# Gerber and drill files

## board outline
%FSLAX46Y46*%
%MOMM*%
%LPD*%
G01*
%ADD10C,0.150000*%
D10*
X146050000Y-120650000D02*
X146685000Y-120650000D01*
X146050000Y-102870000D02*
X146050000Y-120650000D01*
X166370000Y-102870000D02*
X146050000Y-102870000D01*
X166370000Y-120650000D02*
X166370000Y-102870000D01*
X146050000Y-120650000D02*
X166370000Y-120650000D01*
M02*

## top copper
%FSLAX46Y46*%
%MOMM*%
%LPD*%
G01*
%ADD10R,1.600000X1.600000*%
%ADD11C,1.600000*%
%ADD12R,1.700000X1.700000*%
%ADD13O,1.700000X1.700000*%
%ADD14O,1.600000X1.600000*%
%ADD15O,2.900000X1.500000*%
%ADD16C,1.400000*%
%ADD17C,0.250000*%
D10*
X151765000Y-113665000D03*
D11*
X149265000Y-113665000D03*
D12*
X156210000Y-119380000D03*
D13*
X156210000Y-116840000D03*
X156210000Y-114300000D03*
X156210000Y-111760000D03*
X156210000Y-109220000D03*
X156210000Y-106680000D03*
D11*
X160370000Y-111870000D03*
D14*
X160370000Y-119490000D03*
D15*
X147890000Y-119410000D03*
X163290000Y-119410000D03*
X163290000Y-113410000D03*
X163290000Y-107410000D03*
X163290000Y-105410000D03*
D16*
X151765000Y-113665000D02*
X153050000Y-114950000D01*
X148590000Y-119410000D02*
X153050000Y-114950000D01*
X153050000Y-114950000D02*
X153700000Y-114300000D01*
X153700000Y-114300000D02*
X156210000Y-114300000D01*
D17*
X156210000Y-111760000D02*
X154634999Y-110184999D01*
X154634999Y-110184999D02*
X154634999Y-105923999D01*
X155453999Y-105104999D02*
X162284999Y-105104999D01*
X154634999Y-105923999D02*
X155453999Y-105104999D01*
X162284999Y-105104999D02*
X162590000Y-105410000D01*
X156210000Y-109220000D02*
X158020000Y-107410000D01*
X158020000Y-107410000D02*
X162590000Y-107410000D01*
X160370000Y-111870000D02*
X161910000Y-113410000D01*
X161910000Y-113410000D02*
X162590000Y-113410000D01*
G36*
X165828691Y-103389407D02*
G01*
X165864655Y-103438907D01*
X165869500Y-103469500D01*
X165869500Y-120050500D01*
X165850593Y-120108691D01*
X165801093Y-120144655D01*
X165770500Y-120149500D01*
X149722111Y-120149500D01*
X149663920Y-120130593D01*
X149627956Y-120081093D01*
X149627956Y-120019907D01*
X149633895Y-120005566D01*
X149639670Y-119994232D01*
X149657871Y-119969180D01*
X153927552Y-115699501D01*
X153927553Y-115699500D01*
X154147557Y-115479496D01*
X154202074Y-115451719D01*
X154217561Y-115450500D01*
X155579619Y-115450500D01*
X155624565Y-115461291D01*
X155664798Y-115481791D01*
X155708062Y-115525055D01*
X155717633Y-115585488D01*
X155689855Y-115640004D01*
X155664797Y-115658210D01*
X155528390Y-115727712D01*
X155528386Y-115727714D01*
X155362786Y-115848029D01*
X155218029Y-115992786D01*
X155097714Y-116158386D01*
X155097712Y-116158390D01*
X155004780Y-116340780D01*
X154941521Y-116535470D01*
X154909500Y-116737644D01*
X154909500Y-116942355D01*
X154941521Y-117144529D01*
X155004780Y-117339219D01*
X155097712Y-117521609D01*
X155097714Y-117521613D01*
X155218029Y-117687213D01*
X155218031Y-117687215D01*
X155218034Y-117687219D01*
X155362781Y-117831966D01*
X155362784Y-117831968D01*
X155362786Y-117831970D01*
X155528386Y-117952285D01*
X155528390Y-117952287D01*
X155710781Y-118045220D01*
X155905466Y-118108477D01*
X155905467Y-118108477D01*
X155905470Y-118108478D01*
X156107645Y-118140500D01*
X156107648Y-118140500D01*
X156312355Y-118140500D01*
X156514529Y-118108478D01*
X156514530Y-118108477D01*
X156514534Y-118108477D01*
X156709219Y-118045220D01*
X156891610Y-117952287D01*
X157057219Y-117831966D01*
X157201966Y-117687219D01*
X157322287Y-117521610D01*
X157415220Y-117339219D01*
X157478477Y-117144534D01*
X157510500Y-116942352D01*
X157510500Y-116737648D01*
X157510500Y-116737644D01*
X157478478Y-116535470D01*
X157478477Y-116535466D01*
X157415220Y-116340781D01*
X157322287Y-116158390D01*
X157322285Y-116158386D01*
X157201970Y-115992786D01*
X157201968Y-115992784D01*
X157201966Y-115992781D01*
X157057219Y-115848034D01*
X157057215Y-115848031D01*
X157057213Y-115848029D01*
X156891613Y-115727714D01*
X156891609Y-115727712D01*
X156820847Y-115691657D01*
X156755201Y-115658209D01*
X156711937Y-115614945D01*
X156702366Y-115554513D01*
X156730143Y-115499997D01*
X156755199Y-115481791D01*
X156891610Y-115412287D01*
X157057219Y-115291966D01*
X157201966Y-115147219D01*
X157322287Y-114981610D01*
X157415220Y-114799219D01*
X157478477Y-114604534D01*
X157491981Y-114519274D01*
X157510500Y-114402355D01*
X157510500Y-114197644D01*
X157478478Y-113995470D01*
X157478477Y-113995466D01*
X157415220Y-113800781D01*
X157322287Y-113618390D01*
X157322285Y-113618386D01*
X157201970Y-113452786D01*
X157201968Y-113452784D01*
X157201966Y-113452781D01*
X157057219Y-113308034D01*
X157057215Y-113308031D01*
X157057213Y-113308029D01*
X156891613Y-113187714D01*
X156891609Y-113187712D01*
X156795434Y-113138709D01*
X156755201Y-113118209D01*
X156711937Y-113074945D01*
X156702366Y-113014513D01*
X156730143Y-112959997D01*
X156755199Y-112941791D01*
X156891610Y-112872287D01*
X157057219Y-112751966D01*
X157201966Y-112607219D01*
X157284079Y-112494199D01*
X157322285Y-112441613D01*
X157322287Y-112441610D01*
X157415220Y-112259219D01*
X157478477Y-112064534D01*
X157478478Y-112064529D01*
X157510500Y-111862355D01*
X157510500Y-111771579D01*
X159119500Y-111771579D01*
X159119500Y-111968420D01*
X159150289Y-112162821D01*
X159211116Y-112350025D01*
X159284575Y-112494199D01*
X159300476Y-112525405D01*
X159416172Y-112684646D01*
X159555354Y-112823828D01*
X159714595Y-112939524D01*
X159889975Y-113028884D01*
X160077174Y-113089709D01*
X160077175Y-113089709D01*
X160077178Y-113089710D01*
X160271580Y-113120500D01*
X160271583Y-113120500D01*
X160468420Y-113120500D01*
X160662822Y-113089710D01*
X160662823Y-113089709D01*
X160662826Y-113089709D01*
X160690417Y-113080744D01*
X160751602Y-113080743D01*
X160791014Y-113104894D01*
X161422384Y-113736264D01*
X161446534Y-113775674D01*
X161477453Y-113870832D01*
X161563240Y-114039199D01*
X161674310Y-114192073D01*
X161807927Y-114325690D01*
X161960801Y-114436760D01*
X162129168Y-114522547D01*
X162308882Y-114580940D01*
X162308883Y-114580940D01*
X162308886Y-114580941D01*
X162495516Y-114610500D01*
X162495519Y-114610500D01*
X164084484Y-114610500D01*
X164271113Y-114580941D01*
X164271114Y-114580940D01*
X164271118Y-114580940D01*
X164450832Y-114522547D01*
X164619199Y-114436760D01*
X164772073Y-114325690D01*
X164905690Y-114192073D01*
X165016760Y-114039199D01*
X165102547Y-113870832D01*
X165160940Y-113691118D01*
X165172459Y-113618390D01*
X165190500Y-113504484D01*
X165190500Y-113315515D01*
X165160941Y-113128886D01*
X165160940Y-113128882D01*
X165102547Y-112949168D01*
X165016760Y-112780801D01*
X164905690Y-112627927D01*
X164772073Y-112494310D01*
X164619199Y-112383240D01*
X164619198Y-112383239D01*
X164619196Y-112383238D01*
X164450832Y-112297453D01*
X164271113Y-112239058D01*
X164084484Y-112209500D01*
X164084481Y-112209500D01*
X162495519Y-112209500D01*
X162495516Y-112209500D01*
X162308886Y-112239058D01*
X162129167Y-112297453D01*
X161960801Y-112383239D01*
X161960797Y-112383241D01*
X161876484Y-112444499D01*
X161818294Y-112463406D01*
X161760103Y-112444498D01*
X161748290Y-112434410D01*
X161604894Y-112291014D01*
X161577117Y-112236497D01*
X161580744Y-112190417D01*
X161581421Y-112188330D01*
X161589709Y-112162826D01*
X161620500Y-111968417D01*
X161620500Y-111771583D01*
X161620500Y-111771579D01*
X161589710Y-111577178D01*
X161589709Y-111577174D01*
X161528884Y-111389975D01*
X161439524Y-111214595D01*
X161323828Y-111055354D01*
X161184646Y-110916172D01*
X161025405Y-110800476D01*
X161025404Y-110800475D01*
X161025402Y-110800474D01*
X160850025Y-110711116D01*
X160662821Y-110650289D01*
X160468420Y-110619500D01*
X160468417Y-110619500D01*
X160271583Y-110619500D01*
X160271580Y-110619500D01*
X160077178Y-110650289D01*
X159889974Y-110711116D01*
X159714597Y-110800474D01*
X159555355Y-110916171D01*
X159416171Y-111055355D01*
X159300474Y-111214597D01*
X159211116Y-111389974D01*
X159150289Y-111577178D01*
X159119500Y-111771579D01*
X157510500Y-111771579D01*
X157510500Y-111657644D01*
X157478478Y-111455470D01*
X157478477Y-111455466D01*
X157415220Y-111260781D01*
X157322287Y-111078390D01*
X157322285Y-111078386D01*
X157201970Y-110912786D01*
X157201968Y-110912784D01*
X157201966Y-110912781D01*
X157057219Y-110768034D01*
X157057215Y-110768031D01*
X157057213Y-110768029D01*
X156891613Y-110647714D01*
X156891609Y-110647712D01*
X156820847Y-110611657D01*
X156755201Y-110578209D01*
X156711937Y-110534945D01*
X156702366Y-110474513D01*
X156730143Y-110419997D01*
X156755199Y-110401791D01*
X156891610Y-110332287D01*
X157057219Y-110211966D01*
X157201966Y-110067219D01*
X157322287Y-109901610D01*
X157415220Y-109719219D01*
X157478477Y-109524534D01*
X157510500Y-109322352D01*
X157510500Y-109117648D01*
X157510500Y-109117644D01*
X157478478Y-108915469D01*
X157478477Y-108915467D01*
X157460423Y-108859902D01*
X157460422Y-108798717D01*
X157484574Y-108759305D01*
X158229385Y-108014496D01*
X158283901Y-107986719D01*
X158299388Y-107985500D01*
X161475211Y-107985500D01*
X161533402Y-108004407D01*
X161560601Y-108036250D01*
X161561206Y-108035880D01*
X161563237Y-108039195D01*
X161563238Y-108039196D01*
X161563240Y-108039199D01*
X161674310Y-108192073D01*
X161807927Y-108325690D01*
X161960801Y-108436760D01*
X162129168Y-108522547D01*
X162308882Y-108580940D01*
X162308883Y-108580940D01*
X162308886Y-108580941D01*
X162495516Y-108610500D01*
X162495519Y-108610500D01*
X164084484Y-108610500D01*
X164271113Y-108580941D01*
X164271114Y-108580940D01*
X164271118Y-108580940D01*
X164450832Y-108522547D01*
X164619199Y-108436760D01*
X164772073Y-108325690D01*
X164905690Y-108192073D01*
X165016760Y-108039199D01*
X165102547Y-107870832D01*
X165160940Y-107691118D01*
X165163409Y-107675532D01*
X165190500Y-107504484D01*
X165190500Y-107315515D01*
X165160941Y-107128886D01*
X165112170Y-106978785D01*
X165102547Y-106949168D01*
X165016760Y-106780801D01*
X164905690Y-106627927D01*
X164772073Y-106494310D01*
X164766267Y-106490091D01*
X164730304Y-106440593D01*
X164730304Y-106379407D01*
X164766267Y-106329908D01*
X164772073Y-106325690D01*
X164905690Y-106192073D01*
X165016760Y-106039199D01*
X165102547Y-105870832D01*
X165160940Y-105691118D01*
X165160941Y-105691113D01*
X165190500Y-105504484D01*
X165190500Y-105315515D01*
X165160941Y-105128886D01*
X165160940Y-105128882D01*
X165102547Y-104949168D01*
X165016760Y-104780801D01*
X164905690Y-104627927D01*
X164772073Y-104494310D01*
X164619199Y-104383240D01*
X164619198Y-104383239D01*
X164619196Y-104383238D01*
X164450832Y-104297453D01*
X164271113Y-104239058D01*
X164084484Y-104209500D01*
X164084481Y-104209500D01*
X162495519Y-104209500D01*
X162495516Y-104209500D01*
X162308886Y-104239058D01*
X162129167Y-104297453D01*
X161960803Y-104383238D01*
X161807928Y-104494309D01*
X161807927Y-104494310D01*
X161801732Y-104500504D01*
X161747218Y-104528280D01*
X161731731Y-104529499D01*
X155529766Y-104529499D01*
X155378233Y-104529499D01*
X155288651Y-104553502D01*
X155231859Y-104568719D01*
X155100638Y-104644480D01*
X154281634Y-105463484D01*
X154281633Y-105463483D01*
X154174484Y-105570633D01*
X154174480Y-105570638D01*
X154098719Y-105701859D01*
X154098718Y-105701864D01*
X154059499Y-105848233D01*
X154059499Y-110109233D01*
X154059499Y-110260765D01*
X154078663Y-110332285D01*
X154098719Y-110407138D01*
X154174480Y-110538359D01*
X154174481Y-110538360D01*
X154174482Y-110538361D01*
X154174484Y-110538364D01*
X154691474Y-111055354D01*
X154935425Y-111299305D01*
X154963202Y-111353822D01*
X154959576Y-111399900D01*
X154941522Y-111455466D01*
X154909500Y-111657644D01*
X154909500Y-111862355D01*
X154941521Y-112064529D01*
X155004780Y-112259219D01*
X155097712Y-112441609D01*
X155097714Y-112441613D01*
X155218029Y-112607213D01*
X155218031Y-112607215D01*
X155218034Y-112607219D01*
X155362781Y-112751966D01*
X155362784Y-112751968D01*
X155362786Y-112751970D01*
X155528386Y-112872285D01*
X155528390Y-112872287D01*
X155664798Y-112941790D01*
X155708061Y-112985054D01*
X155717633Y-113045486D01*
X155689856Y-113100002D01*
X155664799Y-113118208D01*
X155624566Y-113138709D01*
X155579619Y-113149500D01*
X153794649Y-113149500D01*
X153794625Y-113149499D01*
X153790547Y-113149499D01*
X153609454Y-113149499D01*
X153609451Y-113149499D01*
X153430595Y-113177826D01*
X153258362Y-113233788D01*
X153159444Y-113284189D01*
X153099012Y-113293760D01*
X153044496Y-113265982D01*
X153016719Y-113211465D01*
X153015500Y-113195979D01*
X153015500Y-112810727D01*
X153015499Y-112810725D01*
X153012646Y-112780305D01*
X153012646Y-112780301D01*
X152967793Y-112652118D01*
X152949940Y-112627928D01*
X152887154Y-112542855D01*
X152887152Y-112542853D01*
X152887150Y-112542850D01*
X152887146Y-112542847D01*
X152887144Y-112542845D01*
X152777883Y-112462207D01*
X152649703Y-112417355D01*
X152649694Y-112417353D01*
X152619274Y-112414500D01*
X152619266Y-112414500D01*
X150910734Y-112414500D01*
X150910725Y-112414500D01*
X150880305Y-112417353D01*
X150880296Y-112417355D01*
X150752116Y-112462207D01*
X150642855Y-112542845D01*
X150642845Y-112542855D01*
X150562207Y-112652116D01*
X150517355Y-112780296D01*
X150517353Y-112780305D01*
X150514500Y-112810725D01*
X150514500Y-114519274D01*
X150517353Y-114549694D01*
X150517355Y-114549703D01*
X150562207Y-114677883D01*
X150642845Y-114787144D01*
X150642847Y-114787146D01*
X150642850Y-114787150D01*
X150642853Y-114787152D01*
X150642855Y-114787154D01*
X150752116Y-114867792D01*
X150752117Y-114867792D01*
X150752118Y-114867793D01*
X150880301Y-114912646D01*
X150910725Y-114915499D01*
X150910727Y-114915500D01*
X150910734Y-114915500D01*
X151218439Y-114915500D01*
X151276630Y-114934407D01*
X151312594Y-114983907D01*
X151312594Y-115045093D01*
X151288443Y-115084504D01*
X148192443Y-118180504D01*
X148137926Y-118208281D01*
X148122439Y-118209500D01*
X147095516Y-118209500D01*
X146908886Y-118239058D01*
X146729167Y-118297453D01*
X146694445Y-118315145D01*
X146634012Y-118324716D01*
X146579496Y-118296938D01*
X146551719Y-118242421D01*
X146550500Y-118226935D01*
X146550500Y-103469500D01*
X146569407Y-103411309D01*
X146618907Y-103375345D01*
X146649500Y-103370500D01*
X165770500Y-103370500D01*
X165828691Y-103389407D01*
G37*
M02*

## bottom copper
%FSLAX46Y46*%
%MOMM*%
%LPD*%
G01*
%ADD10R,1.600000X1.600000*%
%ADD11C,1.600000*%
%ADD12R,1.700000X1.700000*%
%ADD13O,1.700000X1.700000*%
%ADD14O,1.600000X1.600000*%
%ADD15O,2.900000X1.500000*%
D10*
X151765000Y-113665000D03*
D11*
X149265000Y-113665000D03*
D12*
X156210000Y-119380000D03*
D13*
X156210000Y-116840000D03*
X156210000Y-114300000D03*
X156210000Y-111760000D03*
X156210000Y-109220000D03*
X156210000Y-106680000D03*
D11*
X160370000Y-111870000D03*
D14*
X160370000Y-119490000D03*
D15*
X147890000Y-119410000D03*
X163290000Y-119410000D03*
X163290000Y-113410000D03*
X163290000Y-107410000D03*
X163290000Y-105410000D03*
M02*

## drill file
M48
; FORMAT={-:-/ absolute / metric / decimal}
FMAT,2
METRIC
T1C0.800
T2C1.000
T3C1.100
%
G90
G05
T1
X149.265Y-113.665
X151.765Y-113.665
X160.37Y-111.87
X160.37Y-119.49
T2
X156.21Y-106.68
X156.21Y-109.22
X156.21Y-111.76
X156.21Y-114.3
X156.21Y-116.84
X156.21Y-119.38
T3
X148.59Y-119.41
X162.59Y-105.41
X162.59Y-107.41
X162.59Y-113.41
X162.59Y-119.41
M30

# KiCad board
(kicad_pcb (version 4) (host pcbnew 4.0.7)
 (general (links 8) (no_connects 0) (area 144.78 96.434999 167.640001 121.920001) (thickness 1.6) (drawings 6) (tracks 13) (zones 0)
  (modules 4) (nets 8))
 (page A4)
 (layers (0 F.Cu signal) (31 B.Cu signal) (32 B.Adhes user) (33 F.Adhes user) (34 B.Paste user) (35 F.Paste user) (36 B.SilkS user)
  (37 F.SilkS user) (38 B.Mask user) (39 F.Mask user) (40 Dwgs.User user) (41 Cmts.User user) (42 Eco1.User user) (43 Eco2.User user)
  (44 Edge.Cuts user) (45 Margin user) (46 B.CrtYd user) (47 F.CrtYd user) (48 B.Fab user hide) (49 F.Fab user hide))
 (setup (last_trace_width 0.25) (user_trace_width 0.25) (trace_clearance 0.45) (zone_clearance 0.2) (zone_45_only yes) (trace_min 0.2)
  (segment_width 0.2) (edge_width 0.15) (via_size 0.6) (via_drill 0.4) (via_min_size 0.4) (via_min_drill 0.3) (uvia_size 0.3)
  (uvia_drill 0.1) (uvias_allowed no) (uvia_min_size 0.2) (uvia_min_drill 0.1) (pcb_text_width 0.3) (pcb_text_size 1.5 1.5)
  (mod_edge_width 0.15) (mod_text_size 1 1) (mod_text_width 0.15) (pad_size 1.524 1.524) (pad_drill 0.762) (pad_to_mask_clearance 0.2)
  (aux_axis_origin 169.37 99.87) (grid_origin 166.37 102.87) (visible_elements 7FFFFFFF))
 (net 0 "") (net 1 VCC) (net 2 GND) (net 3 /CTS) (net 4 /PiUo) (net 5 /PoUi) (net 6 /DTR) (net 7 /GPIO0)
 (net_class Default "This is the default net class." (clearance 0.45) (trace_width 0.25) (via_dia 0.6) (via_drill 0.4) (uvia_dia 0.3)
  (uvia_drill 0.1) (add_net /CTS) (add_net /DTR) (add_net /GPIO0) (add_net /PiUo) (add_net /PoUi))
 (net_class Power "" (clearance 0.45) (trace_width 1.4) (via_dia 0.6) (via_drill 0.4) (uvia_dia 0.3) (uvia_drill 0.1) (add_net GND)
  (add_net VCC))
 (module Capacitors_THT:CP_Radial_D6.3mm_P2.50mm (layer F.Cu) (at 151.765 113.665 180)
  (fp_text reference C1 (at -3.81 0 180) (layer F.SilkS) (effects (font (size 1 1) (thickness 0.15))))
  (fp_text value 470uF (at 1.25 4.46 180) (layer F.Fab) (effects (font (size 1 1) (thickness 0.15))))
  (pad 1 thru_hole rect (at 0 0 180) (size 1.6 1.6) (drill 0.8) (layers *.Cu *.Mask) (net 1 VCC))
  (pad 2 thru_hole circle (at 2.5 0 180) (size 1.6 1.6) (drill 0.8) (layers *.Cu *.Mask) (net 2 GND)))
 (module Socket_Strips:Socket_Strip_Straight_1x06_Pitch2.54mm (layer F.Cu) (at 156.21 119.38 180)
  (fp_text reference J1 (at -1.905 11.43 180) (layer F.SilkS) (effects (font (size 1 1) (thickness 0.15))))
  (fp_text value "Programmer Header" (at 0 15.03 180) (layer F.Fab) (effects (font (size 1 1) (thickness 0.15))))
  (pad 1 thru_hole rect (at 0 0 180) (size 1.7 1.7) (drill 1) (layers *.Cu *.Mask) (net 2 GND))
  (pad 2 thru_hole oval (at 0 2.54 180) (size 1.7 1.7) (drill 1) (layers *.Cu *.Mask) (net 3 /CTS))
  (pad 3 thru_hole oval (at 0 5.08 180) (size 1.7 1.7) (drill 1) (layers *.Cu *.Mask) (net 1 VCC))
  (pad 4 thru_hole oval (at 0 7.62 180) (size 1.7 1.7) (drill 1) (layers *.Cu *.Mask) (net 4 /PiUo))
  (pad 5 thru_hole oval (at 0 10.16 180) (size 1.7 1.7) (drill 1) (layers *.Cu *.Mask) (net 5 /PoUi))
  (pad 6 thru_hole oval (at 0 12.7 180) (size 1.7 1.7) (drill 1) (layers *.Cu *.Mask) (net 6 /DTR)))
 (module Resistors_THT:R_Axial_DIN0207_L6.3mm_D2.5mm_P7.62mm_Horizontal (layer F.Cu) (at 160.37 111.87 270)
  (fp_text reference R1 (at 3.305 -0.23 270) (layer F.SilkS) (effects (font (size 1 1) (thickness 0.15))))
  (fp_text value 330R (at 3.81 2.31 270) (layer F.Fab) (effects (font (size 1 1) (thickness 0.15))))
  (pad 1 thru_hole circle (at 0 0 270) (size 1.6 1.6) (drill 0.8) (layers *.Cu *.Mask) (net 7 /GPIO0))
  (pad 2 thru_hole oval (at 7.62 0 270) (size 1.6 1.6) (drill 0.8) (layers *.Cu *.Mask) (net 2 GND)))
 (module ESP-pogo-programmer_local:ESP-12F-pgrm (layer F.Cu) (at 148.59 105.41)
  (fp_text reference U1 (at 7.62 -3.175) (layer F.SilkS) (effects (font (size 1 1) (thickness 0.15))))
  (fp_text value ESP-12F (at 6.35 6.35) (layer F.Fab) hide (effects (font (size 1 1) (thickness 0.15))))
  (pad 8 thru_hole oval (at 0 14) (size 2.9 1.5) (drill 1.1 (offset -0.7 0)) (layers *.Cu *.Mask F.SilkS) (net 1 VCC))
  (pad 9 thru_hole oval (at 14 14) (size 2.9 1.5) (drill 1.1 (offset 0.7 0)) (layers *.Cu *.Mask F.SilkS) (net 2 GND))
  (pad 12 thru_hole oval (at 14 8) (size 2.9 1.5) (drill 1.1 (offset 0.7 0)) (layers *.Cu *.Mask F.SilkS) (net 7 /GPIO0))
  (pad 15 thru_hole oval (at 14 2) (size 2.9 1.5) (drill 1.1 (offset 0.7 0)) (layers *.Cu *.Mask F.SilkS) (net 5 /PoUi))
  (pad 16 thru_hole oval (at 14 0) (size 2.9 1.5) (drill 1.1 (offset 0.7 0)) (layers *.Cu *.Mask F.SilkS) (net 4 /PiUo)))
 (gr_line (start 146.05 120.65) (end 146.685 120.65) (angle 90) (layer Edge.Cuts) (width 0.15))
 (gr_line (start 146.05 102.87) (end 146.05 120.65) (angle 90) (layer Edge.Cuts) (width 0.15))
 (gr_line (start 166.37 102.87) (end 146.05 102.87) (angle 90) (layer Edge.Cuts) (width 0.15))
 (gr_line (start 166.37 120.65) (end 166.37 102.87) (angle 90) (layer Edge.Cuts) (width 0.15))
 (gr_line (start 146.05 120.65) (end 166.37 120.65) (angle 90) (layer Edge.Cuts) (width 0.15))
 (segment (start 151.765 113.665) (end 153.05 114.95) (width 1.4) (layer F.Cu) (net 1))
 (segment (start 148.59 119.41) (end 153.05 114.95) (width 1.4) (layer F.Cu) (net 1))
 (segment (start 153.05 114.95) (end 153.7 114.3) (width 1.4) (layer F.Cu) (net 1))
 (segment (start 153.7 114.3) (end 156.21 114.3) (width 1.4) (layer F.Cu) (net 1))
 (segment (start 156.21 111.76) (end 154.634999 110.184999) (width 0.25) (layer F.Cu) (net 4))
 (segment (start 154.634999 110.184999) (end 154.634999 105.923999) (width 0.25) (layer F.Cu) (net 4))
 (segment (start 155.453999 105.104999) (end 162.284999 105.104999) (width 0.25) (layer F.Cu) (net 4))
 (segment (start 154.634999 105.923999) (end 155.453999 105.104999) (width 0.25) (layer F.Cu) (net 4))
 (segment (start 162.284999 105.104999) (end 162.59 105.41) (width 0.25) (layer F.Cu) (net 4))
 (segment (start 156.21 109.22) (end 158.02 107.41) (width 0.25) (layer F.Cu) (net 5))
 (segment (start 158.02 107.41) (end 162.59 107.41) (width 0.25) (layer F.Cu) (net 5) (status 20))
 (segment (start 160.37 111.87) (end 161.91 113.41) (width 0.25) (layer F.Cu) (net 7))
 (segment (start 161.91 113.41) (end 162.59 113.41) (width 0.25) (layer F.Cu) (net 7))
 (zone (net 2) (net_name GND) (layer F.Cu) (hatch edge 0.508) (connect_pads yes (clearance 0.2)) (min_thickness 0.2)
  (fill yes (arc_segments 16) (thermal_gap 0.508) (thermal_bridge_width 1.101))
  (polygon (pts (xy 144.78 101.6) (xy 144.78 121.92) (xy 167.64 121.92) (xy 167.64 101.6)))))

